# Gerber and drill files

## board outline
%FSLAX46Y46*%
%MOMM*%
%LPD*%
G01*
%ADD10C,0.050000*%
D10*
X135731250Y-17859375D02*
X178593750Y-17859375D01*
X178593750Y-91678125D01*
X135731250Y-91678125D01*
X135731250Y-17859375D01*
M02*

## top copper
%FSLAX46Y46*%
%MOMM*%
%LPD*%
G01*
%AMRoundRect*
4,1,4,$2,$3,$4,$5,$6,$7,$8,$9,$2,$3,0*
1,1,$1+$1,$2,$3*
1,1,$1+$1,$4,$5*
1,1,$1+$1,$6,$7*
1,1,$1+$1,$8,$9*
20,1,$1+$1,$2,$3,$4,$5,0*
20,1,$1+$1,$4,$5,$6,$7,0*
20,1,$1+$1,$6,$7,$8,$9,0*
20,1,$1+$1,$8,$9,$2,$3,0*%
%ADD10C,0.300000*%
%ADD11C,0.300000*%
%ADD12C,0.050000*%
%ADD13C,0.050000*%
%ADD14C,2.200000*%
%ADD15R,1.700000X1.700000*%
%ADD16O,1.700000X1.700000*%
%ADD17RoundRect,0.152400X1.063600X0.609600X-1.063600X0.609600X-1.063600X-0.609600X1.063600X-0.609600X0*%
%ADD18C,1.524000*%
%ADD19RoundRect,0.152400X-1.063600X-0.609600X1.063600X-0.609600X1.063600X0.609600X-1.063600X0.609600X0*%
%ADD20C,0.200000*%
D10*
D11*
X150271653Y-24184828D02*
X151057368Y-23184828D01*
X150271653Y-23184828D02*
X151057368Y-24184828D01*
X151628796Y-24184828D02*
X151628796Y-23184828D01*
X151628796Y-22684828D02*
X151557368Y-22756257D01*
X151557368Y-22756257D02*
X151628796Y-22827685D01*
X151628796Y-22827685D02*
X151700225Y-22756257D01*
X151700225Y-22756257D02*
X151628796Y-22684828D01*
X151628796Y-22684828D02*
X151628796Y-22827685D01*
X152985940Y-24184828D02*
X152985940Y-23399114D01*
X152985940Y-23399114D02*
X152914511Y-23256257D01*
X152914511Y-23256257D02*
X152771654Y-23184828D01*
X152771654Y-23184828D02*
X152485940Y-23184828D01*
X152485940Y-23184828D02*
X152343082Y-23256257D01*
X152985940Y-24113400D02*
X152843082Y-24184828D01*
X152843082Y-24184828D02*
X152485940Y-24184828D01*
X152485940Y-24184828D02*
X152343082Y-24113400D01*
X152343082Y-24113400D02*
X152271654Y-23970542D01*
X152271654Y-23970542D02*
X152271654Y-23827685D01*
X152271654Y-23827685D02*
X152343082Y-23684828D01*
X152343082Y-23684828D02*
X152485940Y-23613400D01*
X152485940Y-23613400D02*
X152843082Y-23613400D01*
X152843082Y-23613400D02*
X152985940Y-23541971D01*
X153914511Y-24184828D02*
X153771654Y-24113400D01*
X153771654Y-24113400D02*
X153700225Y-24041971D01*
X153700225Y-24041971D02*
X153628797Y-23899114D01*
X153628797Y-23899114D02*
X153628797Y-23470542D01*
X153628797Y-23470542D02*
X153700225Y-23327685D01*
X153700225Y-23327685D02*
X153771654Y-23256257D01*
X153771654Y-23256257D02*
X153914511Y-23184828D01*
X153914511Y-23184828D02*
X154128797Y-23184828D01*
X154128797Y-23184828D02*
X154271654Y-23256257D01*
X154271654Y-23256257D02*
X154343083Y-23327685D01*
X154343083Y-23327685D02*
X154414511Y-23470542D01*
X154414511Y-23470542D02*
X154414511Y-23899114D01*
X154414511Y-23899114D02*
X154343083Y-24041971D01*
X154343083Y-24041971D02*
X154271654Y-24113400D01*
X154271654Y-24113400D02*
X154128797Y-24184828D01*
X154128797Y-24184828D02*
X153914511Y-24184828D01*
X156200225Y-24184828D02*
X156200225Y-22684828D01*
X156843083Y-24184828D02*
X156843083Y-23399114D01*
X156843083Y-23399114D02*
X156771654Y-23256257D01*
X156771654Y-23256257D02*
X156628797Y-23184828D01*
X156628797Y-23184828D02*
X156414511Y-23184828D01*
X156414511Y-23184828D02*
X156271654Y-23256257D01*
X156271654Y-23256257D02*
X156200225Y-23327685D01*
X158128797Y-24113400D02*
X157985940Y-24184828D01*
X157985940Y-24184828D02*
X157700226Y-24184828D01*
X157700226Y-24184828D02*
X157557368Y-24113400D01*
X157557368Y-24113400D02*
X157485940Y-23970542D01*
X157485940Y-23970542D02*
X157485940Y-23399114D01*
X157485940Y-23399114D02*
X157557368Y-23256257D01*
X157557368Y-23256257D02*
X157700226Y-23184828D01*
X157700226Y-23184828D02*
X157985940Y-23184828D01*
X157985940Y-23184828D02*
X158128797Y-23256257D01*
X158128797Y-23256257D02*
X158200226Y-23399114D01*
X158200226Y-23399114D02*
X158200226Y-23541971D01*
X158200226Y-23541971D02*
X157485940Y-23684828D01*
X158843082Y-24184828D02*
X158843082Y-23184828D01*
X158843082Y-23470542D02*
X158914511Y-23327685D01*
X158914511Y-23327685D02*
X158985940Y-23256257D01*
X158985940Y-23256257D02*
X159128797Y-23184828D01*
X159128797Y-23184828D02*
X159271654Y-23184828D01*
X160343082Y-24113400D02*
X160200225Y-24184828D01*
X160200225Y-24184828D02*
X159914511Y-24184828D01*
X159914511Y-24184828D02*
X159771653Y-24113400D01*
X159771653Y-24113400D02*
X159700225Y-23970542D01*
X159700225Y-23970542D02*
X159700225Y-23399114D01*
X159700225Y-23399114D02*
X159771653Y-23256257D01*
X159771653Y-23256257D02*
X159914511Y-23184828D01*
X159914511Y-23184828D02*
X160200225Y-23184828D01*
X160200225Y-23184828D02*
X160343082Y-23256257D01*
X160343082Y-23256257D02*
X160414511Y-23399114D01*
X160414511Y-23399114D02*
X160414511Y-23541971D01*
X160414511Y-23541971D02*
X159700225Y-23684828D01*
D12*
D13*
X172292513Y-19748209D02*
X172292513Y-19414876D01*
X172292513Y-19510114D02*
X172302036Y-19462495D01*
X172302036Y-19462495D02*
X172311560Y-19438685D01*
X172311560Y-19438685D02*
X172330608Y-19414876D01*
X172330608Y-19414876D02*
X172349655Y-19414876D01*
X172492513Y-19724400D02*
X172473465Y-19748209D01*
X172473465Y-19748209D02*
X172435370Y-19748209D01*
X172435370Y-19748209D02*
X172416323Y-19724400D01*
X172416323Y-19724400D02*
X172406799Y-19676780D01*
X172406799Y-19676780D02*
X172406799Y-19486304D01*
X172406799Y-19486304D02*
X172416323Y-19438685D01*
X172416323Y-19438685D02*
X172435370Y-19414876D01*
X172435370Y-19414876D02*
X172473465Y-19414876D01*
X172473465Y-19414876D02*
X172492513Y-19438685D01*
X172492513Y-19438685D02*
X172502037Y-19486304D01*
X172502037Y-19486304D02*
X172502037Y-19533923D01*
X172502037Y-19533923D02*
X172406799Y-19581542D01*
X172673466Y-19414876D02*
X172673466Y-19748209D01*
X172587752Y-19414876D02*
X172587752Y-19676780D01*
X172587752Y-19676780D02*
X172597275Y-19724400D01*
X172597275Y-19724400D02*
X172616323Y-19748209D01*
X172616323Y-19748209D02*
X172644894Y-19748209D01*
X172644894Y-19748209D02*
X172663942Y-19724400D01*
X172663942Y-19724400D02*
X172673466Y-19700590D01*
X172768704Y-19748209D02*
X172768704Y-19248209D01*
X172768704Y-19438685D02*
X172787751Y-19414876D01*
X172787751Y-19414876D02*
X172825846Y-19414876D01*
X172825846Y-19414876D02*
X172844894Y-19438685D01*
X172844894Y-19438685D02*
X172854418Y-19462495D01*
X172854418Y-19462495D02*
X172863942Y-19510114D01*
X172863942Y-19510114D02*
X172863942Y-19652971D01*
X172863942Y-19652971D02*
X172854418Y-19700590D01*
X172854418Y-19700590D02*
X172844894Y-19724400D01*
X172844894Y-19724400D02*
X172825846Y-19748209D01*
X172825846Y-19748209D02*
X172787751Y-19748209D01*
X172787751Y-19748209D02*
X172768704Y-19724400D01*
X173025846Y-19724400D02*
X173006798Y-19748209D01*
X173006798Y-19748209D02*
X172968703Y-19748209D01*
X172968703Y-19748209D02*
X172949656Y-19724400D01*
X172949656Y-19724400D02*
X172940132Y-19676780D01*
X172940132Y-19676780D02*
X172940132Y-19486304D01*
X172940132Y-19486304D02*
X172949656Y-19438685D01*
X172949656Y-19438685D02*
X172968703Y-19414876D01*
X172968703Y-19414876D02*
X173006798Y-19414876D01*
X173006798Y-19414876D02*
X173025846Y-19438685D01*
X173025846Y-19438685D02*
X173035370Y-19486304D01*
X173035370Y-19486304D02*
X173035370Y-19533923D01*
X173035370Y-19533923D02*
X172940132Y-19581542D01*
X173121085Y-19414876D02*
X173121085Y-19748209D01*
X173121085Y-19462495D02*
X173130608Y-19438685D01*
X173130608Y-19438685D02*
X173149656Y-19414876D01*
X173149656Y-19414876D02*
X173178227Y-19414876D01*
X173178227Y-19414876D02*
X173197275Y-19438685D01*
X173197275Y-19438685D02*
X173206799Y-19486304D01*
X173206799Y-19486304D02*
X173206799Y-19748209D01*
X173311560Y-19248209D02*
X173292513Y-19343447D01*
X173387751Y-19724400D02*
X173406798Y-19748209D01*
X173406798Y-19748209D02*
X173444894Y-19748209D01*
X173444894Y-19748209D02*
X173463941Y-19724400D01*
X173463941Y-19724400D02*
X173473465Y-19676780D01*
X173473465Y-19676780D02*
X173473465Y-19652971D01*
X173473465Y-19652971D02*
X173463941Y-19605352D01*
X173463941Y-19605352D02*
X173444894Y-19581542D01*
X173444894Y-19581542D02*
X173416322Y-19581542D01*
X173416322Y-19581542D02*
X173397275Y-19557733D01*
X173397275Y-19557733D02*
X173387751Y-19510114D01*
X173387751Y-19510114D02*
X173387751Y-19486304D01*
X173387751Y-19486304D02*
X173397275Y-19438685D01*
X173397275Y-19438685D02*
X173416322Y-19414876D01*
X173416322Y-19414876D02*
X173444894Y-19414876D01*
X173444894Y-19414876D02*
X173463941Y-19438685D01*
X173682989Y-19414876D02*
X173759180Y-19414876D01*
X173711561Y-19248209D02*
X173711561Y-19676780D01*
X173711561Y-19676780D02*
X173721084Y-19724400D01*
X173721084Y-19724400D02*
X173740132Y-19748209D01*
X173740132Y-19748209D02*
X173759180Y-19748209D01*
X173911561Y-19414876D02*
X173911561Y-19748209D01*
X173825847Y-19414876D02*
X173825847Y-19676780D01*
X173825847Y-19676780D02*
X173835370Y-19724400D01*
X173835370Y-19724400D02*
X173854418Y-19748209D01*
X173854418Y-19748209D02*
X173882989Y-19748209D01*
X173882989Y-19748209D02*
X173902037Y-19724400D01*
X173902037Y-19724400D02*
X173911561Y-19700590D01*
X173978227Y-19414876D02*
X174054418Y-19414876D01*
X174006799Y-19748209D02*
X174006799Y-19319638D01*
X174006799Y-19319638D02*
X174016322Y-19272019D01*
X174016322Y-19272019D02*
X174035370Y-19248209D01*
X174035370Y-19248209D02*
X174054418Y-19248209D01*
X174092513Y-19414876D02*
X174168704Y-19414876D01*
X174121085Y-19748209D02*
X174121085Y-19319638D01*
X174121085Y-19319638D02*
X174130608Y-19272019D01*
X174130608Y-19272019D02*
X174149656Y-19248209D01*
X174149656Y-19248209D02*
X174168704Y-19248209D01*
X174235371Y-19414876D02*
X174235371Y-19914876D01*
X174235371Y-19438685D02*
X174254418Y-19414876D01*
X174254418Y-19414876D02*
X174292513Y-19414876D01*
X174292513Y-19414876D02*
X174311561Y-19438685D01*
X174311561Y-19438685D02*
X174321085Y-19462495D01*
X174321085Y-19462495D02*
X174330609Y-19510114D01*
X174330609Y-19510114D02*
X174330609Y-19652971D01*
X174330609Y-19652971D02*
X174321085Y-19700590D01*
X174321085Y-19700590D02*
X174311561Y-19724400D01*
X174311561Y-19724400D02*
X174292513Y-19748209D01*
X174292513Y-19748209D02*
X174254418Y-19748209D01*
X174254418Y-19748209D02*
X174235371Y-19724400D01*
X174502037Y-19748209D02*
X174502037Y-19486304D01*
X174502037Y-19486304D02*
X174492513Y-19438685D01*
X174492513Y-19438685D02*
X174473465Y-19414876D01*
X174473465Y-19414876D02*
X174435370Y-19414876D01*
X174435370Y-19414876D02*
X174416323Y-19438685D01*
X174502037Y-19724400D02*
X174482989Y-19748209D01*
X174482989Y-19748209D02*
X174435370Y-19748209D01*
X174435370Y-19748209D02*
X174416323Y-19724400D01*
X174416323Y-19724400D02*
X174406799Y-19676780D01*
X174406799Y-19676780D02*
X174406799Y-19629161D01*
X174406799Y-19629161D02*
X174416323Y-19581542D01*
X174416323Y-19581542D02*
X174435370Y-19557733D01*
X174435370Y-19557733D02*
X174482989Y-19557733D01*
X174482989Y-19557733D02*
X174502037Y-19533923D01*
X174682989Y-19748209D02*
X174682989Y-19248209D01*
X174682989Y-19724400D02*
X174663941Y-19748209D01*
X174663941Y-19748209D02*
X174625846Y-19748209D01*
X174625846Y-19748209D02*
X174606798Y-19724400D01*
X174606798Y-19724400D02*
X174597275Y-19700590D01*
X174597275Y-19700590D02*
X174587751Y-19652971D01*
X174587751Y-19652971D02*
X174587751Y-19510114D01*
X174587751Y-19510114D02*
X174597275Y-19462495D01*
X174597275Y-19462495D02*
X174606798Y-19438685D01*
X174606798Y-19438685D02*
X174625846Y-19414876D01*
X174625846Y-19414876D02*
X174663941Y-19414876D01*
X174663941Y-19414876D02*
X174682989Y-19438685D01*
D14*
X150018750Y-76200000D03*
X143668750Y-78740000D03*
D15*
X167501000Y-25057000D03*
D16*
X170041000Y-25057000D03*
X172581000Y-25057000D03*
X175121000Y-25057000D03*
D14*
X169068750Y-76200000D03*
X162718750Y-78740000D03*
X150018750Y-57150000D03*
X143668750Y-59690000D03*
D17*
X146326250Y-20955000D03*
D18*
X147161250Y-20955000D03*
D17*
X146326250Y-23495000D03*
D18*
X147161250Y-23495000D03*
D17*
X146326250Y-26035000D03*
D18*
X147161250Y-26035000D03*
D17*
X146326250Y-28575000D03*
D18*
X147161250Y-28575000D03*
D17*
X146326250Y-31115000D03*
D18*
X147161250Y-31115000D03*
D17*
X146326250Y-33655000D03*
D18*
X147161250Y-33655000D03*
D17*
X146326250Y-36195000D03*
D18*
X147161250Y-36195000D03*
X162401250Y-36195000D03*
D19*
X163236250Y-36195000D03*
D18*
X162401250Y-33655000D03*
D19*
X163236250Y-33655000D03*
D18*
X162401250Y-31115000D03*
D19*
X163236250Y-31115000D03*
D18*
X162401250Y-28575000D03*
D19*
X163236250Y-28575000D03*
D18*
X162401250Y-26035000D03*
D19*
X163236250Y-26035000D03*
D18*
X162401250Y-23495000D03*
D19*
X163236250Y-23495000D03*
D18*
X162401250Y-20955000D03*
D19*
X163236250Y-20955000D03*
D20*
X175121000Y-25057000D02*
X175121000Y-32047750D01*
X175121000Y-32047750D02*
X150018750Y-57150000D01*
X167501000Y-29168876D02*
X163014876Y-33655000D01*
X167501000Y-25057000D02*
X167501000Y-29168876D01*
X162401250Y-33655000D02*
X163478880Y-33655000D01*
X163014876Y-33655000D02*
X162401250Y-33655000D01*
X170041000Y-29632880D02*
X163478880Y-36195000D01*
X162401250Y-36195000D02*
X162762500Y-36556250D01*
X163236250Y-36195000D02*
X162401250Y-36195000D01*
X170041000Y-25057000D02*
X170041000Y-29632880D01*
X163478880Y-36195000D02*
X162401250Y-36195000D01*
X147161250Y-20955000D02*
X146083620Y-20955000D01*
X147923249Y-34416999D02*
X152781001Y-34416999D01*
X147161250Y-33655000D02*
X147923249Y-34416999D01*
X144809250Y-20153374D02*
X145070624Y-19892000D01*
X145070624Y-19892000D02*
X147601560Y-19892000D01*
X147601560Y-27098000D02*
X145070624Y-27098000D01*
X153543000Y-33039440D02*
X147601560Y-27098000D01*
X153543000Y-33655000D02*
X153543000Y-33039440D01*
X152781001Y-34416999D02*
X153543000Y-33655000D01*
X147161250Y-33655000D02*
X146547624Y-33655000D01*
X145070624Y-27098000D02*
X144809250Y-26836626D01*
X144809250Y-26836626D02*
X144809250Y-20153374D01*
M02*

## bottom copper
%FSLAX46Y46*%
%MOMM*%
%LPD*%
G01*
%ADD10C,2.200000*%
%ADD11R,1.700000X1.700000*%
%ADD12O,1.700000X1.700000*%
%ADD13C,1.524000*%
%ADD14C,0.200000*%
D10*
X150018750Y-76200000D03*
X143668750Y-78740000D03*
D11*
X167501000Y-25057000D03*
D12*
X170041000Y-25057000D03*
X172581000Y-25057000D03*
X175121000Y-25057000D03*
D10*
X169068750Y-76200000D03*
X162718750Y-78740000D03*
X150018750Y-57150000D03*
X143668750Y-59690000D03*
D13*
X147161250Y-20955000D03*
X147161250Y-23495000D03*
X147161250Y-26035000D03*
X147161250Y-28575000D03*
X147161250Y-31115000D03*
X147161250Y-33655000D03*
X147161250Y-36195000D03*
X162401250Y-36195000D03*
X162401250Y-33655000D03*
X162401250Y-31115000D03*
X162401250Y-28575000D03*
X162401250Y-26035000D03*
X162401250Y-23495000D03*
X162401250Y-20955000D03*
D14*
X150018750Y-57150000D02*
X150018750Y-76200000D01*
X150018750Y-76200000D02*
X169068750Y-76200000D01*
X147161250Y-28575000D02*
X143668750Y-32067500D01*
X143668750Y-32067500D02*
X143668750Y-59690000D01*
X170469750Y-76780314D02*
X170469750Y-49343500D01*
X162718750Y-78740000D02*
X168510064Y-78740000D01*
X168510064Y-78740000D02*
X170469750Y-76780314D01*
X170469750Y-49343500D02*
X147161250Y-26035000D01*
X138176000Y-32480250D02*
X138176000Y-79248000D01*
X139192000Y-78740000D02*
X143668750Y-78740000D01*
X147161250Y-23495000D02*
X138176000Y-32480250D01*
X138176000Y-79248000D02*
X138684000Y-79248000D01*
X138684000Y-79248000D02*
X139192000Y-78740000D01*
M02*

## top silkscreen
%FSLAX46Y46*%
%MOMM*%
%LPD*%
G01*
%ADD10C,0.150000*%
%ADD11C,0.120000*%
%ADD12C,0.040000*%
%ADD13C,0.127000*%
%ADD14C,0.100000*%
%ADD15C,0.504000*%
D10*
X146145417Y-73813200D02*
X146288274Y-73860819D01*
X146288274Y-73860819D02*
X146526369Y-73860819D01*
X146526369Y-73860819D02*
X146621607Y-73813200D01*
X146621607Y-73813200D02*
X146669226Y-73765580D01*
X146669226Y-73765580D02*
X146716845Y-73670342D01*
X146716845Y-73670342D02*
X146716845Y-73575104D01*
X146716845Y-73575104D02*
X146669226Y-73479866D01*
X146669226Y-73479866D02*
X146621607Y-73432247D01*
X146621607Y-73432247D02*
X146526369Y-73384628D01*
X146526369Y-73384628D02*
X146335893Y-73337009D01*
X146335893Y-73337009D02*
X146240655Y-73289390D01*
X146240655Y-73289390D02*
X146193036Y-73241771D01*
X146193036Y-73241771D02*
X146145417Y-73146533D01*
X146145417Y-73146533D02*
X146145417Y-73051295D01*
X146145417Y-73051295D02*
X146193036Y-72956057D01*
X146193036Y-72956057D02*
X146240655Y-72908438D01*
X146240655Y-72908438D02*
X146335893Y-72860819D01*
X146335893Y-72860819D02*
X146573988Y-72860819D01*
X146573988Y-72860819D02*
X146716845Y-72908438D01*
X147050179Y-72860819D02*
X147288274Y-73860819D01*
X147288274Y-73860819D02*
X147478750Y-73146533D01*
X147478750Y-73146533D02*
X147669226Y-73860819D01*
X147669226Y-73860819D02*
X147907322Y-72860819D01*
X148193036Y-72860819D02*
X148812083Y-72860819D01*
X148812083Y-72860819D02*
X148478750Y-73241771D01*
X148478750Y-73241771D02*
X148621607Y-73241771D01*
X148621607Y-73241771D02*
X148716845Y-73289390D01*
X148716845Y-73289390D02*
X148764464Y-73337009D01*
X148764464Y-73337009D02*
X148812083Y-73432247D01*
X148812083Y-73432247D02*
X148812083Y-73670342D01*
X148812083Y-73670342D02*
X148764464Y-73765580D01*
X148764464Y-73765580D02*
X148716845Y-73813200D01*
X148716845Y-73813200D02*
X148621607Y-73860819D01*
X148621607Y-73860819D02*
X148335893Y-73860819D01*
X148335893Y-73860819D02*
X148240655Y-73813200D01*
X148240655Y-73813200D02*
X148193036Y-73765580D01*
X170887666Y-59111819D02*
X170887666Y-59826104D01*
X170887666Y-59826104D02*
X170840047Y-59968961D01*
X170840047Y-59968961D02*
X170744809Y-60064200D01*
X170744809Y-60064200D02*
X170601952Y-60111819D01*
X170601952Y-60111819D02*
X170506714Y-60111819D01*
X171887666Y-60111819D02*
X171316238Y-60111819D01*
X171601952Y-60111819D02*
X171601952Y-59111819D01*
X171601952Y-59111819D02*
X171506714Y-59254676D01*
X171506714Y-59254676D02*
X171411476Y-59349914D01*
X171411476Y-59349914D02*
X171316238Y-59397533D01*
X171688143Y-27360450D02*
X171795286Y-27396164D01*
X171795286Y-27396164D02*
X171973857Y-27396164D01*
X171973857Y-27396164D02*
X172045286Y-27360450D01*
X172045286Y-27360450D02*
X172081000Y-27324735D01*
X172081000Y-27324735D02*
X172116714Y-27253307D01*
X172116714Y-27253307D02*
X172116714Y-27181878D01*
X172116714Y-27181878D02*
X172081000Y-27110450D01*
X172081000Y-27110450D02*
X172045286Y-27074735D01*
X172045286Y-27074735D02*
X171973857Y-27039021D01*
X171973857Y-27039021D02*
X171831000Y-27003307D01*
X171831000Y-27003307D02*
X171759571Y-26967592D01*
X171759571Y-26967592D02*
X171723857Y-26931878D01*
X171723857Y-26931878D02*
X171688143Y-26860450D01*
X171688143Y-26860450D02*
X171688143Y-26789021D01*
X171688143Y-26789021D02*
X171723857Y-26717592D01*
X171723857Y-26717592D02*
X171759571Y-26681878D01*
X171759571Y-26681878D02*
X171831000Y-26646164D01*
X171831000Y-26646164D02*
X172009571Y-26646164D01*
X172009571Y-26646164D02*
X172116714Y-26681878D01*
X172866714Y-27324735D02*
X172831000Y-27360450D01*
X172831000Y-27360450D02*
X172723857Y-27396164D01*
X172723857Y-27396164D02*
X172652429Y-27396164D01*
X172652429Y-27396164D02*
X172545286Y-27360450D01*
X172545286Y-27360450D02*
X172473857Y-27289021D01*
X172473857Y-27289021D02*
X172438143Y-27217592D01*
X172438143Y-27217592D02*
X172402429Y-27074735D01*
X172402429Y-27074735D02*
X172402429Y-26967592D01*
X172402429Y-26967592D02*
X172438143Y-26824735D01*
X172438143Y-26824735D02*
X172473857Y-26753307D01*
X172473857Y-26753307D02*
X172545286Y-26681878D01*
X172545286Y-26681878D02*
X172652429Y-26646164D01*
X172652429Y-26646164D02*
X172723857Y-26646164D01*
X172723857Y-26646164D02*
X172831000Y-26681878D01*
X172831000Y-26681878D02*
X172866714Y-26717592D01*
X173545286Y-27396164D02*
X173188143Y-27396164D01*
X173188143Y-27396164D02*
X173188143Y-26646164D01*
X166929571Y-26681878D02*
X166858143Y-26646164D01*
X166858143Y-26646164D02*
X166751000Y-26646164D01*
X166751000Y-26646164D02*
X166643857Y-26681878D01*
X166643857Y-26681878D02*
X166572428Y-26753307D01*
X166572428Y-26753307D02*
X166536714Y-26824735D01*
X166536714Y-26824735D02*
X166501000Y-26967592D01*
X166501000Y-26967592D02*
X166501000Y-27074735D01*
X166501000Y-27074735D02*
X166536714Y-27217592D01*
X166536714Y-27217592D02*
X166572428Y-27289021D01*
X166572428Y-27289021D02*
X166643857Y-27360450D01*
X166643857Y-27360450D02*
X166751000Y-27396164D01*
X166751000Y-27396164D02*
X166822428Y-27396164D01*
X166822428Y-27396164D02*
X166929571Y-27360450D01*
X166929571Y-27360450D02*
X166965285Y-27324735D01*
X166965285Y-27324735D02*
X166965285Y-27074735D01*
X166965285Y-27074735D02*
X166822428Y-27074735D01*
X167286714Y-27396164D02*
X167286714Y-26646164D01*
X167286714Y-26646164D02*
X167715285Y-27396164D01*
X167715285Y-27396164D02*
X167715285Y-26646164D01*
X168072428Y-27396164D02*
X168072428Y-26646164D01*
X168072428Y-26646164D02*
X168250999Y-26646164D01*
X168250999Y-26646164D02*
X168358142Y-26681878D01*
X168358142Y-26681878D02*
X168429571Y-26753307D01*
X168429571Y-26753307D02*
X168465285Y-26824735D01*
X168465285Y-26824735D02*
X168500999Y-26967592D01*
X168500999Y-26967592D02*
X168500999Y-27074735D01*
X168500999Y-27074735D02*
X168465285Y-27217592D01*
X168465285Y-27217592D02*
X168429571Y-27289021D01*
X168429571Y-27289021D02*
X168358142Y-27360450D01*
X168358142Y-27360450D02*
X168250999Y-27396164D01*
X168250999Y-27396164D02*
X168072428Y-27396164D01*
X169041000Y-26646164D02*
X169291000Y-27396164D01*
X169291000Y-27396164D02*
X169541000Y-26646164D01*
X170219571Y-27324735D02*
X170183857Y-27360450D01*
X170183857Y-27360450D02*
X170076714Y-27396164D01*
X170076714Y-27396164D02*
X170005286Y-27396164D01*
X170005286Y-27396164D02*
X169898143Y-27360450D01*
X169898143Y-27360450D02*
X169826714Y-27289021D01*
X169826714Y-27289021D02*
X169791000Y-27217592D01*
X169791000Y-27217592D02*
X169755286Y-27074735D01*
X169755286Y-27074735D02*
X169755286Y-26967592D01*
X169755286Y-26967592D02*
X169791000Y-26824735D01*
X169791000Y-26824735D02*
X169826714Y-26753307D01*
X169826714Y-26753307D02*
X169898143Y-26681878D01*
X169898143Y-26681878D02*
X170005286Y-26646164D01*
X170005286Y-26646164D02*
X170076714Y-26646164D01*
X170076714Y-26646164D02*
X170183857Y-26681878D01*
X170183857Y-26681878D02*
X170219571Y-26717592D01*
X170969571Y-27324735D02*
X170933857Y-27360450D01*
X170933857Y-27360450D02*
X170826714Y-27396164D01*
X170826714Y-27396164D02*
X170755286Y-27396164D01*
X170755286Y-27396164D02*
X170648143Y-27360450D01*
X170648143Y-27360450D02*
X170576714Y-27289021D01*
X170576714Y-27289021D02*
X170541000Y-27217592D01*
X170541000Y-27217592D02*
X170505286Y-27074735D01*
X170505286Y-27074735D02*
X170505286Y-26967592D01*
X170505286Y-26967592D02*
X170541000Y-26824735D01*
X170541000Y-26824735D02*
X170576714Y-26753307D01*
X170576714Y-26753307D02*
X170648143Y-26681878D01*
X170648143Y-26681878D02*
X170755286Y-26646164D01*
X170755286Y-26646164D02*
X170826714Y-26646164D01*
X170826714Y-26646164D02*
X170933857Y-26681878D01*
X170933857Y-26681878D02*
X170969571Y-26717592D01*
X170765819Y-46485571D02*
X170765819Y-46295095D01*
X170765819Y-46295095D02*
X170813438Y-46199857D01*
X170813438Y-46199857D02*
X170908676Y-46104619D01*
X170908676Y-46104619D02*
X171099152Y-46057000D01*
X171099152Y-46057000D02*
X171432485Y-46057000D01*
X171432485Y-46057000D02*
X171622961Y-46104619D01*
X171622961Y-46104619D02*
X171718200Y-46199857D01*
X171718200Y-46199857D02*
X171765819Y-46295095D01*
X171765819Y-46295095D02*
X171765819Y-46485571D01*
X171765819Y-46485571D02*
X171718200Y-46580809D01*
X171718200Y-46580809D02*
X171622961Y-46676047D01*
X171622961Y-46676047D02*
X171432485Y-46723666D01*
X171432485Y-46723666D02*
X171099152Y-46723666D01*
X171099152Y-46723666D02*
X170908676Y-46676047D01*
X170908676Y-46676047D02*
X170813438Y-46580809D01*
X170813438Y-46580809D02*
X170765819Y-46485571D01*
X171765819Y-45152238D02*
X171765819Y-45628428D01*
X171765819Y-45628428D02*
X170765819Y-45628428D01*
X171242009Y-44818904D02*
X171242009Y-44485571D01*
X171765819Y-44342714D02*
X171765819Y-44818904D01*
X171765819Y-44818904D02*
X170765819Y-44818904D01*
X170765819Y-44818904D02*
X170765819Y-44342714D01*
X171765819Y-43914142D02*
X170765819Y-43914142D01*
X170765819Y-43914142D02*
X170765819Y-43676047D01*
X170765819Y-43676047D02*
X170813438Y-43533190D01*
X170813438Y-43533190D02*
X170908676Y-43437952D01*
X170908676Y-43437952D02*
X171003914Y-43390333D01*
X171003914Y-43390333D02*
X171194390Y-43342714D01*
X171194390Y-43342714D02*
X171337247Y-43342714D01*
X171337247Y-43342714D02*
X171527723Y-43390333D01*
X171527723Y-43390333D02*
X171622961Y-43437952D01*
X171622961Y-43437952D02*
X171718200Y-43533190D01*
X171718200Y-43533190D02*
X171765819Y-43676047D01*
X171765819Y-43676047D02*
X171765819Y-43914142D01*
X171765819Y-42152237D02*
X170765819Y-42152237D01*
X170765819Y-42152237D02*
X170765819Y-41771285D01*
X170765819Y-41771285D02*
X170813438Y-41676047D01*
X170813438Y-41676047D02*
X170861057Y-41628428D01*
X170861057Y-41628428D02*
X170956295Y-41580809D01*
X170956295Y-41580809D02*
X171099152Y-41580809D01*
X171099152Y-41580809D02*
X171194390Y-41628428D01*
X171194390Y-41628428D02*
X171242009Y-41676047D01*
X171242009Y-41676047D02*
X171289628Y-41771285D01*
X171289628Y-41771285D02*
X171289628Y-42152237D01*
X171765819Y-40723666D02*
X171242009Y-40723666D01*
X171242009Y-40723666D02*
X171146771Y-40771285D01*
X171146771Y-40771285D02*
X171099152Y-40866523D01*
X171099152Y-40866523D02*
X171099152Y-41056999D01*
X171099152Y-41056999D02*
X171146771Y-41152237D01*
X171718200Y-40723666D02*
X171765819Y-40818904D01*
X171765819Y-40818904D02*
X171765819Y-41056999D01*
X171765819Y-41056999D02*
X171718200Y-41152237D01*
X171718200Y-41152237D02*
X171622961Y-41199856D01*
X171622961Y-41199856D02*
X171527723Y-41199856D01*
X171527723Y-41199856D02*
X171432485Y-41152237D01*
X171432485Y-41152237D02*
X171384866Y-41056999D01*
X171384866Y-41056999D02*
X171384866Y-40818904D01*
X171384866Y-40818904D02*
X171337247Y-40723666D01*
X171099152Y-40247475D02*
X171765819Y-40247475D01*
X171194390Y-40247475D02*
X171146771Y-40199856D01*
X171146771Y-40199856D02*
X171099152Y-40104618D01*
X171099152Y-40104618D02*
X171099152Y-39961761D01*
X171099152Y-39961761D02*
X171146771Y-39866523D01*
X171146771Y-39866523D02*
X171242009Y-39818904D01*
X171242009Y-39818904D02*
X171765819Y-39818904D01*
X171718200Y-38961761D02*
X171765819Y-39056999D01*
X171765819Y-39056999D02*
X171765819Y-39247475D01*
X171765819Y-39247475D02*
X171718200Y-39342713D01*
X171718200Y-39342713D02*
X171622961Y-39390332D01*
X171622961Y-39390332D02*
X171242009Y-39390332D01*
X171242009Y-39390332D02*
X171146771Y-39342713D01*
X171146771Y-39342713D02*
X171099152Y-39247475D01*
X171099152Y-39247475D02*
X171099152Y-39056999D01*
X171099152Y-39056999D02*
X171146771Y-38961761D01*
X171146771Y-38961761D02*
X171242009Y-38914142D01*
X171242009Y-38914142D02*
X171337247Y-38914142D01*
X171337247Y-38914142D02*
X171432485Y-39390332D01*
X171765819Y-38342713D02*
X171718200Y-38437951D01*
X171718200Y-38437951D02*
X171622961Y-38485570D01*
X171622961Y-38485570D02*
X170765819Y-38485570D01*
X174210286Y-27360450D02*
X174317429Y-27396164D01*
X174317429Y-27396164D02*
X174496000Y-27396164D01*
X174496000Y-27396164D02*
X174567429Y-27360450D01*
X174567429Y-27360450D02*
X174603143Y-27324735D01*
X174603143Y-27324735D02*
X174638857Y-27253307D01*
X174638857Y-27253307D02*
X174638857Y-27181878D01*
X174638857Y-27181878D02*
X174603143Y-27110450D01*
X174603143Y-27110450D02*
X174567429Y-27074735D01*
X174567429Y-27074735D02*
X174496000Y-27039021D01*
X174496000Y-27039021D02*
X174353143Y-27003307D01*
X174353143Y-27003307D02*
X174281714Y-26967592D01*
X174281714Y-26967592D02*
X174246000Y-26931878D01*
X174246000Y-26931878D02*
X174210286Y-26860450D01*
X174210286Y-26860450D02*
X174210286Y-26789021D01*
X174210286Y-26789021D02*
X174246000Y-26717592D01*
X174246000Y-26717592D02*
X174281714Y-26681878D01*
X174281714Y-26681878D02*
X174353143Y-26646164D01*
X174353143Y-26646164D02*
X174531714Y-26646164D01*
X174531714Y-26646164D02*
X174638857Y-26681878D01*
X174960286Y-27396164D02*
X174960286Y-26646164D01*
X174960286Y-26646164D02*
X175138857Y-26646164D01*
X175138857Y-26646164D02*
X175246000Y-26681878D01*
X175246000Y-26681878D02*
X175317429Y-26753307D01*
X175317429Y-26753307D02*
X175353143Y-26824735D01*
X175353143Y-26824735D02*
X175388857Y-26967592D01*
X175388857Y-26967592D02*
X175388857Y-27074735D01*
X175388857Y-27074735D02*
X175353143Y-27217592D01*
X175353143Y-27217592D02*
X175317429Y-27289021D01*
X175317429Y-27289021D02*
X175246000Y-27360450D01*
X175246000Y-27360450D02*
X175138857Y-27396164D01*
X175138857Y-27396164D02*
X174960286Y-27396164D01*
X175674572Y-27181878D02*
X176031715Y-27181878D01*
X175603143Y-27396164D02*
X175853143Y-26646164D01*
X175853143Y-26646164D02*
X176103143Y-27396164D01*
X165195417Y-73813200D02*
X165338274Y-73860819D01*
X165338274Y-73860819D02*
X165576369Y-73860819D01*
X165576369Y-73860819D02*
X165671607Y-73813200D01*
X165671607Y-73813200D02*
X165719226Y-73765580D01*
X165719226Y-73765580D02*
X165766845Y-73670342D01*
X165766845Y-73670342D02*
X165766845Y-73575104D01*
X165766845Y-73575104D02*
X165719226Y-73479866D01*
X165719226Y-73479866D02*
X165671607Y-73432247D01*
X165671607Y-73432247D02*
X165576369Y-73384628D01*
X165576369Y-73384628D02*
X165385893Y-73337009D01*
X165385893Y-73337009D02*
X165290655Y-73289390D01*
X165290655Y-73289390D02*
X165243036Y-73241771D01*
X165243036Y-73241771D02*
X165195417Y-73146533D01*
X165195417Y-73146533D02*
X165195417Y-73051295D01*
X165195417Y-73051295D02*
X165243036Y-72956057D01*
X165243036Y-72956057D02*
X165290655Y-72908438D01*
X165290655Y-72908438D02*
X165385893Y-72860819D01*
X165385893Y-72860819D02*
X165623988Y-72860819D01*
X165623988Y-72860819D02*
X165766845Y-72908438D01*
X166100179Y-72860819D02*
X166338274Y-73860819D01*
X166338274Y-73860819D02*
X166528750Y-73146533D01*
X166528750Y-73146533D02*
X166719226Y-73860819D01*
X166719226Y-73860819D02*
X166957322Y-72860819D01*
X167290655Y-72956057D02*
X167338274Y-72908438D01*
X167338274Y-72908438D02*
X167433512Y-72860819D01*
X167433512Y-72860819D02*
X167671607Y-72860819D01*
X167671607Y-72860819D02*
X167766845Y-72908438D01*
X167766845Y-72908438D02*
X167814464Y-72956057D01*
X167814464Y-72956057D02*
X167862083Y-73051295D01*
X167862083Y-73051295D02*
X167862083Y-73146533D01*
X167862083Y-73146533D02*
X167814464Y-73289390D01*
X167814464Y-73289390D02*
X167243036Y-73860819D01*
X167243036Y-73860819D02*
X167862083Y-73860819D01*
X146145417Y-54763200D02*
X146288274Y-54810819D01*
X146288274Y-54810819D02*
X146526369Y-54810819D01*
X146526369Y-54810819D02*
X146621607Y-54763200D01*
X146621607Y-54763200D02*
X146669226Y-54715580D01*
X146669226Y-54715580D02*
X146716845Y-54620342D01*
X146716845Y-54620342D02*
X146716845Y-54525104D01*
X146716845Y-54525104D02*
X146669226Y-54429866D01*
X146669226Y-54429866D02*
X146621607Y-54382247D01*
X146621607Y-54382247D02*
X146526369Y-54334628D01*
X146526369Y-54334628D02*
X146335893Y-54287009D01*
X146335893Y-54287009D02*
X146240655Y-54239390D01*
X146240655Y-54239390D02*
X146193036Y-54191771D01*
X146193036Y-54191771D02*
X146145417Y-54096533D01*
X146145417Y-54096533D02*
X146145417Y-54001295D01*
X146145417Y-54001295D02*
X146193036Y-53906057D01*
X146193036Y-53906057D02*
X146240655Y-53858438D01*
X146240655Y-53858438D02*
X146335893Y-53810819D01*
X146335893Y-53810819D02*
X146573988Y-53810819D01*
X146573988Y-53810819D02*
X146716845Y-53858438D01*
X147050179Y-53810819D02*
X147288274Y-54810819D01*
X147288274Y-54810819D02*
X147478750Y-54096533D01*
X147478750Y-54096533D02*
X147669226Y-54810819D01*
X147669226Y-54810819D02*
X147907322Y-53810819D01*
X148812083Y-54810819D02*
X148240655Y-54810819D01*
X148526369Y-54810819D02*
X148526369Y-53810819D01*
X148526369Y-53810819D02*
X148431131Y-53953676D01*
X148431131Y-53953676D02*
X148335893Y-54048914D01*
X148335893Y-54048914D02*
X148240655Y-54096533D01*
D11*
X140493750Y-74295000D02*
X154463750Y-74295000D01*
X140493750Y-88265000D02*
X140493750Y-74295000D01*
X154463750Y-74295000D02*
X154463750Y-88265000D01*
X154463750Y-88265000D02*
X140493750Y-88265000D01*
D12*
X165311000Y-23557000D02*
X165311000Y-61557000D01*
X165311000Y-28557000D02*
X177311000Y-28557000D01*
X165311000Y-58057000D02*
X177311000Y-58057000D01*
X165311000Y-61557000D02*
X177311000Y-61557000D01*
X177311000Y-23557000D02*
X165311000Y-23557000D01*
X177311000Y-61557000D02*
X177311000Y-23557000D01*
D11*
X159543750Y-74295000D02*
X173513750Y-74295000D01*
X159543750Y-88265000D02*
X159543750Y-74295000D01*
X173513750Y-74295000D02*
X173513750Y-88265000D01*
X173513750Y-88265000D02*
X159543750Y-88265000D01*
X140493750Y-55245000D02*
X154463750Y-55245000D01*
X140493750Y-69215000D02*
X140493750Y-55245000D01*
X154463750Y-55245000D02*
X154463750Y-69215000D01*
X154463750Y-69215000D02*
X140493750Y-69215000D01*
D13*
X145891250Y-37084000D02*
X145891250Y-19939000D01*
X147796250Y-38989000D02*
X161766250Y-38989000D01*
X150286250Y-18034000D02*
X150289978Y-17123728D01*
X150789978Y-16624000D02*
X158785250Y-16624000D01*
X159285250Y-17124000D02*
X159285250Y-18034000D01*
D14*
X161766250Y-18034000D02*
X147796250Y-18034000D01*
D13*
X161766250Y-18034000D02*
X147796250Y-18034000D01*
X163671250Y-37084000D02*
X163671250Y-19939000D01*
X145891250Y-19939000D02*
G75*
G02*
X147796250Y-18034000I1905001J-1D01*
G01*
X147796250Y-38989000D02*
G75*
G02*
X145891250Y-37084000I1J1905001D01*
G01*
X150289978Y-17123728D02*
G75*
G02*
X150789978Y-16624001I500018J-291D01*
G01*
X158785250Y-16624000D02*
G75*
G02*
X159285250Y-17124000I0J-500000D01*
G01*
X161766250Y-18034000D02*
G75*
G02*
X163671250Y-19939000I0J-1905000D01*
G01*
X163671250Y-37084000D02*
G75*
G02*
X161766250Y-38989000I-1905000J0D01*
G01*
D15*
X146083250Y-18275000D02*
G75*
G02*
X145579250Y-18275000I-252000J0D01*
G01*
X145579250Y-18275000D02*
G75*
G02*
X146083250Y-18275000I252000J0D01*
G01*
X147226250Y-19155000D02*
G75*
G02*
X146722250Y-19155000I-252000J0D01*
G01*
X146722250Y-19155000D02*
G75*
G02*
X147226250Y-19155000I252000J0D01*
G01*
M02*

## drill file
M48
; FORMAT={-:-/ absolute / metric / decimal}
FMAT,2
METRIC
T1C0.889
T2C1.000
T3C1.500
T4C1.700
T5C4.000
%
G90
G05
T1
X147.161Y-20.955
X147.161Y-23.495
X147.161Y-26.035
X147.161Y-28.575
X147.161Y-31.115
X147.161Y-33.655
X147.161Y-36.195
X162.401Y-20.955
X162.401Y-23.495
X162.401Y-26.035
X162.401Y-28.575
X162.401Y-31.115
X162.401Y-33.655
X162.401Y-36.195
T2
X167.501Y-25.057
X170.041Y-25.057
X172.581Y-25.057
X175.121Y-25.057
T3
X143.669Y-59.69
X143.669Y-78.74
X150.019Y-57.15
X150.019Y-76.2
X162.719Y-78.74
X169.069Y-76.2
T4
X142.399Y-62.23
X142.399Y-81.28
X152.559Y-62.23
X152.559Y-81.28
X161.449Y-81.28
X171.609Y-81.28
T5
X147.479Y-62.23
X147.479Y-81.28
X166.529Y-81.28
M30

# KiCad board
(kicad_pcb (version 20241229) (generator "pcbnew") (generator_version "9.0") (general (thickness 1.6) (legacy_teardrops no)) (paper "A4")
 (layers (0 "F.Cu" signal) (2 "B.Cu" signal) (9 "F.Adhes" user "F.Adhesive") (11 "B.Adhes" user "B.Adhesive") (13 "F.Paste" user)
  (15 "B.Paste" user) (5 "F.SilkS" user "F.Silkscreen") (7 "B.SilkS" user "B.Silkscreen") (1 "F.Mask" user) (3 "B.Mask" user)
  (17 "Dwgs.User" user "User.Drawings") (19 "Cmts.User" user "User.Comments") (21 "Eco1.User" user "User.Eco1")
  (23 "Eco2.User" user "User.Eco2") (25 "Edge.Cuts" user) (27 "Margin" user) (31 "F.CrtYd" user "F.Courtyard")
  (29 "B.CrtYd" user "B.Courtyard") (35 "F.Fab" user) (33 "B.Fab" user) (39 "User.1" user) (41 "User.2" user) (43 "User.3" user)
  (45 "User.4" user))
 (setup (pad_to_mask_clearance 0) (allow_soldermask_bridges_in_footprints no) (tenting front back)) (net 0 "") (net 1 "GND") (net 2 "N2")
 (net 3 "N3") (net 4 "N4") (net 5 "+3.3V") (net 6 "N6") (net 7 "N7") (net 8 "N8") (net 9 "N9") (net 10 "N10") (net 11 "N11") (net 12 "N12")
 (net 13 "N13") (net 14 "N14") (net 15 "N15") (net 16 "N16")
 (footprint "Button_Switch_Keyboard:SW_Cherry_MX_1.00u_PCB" (layer "F.Cu") (at 150.01875 76.2)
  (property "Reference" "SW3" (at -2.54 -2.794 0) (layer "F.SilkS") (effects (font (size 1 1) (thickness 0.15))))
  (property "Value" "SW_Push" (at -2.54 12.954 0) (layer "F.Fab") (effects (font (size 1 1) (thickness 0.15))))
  (fp_line (start -9.525 -1.905) (end 4.445 -1.905) (stroke (width 0.12) (type solid)) (layer "F.SilkS"))
  (fp_line (start -9.525 12.065) (end -9.525 -1.905) (stroke (width 0.12) (type solid)) (layer "F.SilkS"))
  (fp_line (start 4.445 -1.905) (end 4.445 12.065) (stroke (width 0.12) (type solid)) (layer "F.SilkS"))
  (fp_line (start 4.445 12.065) (end -9.525 12.065) (stroke (width 0.12) (type solid)) (layer "F.SilkS"))
  (pad "" np_thru_hole circle (at -7.62 5.08) (size 1.7 1.7) (drill 1.7) (layers "*.Cu" "*.Mask"))
  (pad "" np_thru_hole circle (at -2.54 5.08) (size 4 4) (drill 4) (layers "*.Cu" "*.Mask"))
  (pad "" np_thru_hole circle (at 2.54 5.08) (size 1.7 1.7) (drill 1.7) (layers "*.Cu" "*.Mask"))
  (pad "1" thru_hole circle (at 0 0) (size 2.2 2.2) (drill 1.5) (layers "*.Cu" "*.Mask") (remove_unused_layers no) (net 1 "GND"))
  (pad "2" thru_hole circle (at -6.35 2.54) (size 2.2 2.2) (drill 1.5) (layers "*.Cu" "*.Mask") (remove_unused_layers no) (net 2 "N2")))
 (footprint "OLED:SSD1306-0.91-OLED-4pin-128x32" (layer "F.Cu") (at 165.311 61.557 90)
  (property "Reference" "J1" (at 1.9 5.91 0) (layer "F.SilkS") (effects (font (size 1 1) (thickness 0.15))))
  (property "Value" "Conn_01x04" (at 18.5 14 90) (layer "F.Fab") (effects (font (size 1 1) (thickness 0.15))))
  (fp_line (start 38 0) (end 0 0) (stroke (width 0.04) (type solid)) (layer "F.SilkS"))
  (fp_line (start 33 0) (end 33 12) (stroke (width 0.04) (type solid)) (layer "F.SilkS"))
  (fp_line (start 3.5 0) (end 3.5 12) (stroke (width 0.04) (type solid)) (layer "F.SilkS"))
  (fp_line (start 0 0) (end 0 12) (stroke (width 0.04) (type solid)) (layer "F.SilkS"))
  (fp_line (start 38 12) (end 38 0) (stroke (width 0.04) (type solid)) (layer "F.SilkS"))
  (fp_line (start 0 12) (end 38 12) (stroke (width 0.04) (type solid)) (layer "F.SilkS"))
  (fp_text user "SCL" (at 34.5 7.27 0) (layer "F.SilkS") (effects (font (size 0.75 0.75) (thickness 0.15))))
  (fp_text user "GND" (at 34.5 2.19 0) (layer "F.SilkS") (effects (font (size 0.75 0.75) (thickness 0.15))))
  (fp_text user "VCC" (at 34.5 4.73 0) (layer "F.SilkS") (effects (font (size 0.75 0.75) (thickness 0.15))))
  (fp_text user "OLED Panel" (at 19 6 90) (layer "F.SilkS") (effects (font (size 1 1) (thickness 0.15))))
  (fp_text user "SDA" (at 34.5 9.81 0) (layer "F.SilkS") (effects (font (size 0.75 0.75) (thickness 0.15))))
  (pad "1" thru_hole rect (at 36.5 2.19 90) (size 1.7 1.7) (drill 1) (layers "*.Cu" "*.Mask") (remove_unused_layers no) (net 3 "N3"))
  (pad "2" thru_hole oval (at 36.5 4.73 90) (size 1.7 1.7) (drill 1) (layers "*.Cu" "*.Mask") (remove_unused_layers no) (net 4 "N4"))
  (pad "3" thru_hole oval (at 36.5 7.27 90) (size 1.7 1.7) (drill 1) (layers "*.Cu" "*.Mask") (remove_unused_layers no) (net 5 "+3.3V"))
  (pad "4" thru_hole oval (at 36.5 9.81 90) (size 1.7 1.7) (drill 1) (layers "*.Cu" "*.Mask") (remove_unused_layers no) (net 1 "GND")))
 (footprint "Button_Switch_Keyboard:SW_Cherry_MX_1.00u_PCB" (layer "F.Cu") (at 169.06875 76.2)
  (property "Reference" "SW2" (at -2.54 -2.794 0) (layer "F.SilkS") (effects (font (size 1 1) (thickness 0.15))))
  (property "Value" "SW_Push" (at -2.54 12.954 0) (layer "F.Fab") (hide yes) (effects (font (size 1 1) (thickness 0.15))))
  (fp_line (start -9.525 -1.905) (end 4.445 -1.905) (stroke (width 0.12) (type solid)) (layer "F.SilkS"))
  (fp_line (start -9.525 12.065) (end -9.525 -1.905) (stroke (width 0.12) (type solid)) (layer "F.SilkS"))
  (fp_line (start 4.445 -1.905) (end 4.445 12.065) (stroke (width 0.12) (type solid)) (layer "F.SilkS"))
  (fp_line (start 4.445 12.065) (end -9.525 12.065) (stroke (width 0.12) (type solid)) (layer "F.SilkS"))
  (pad "" np_thru_hole circle (at -7.62 5.08) (size 1.7 1.7) (drill 1.7) (layers "*.Cu" "*.Mask"))
  (pad "" np_thru_hole circle (at -2.54 5.08) (size 4 4) (drill 4) (layers "*.Cu" "*.Mask"))
  (pad "" np_thru_hole circle (at 2.54 5.08) (size 1.7 1.7) (drill 1.7) (layers "*.Cu" "*.Mask"))
  (pad "1" thru_hole circle (at 0 0) (size 2.2 2.2) (drill 1.5) (layers "*.Cu" "*.Mask") (remove_unused_layers no) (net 1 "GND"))
  (pad "2" thru_hole circle (at -6.35 2.54) (size 2.2 2.2) (drill 1.5) (layers "*.Cu" "*.Mask") (remove_unused_layers no) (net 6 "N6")))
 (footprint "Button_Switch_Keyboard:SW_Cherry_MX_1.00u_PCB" (layer "F.Cu") (at 150.01875 57.15)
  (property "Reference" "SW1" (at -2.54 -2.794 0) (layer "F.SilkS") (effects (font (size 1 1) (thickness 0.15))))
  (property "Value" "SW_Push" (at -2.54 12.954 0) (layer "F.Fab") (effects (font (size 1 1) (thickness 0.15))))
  (fp_line (start -9.525 -1.905) (end 4.445 -1.905) (stroke (width 0.12) (type solid)) (layer "F.SilkS"))
  (fp_line (start -9.525 12.065) (end -9.525 -1.905) (stroke (width 0.12) (type solid)) (layer "F.SilkS"))
  (fp_line (start 4.445 -1.905) (end 4.445 12.065) (stroke (width 0.12) (type solid)) (layer "F.SilkS"))
  (fp_line (start 4.445 12.065) (end -9.525 12.065) (stroke (width 0.12) (type solid)) (layer "F.SilkS"))
  (pad "" np_thru_hole circle (at -7.62 5.08) (size 1.7 1.7) (drill 1.7) (layers "*.Cu" "*.Mask"))
  (pad "" np_thru_hole circle (at -2.54 5.08) (size 4 4) (drill 4) (layers "*.Cu" "*.Mask"))
  (pad "" np_thru_hole circle (at 2.54 5.08) (size 1.7 1.7) (drill 1.7) (layers "*.Cu" "*.Mask"))
  (pad "1" thru_hole circle (at 0 0) (size 2.2 2.2) (drill 1.5) (layers "*.Cu" "*.Mask") (remove_unused_layers no) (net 1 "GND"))
  (pad "2" thru_hole circle (at -6.35 2.54) (size 2.2 2.2) (drill 1.5) (layers "*.Cu" "*.Mask") (remove_unused_layers no) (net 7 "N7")))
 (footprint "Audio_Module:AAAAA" (layer "F.Cu") (at 154.78125 28.575)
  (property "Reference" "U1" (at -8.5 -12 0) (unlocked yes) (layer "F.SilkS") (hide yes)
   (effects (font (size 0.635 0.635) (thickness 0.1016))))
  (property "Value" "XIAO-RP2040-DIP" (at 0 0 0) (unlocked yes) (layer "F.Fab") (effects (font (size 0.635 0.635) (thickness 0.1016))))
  (fp_line (start -8.89 8.509) (end -8.89 -8.636) (stroke (width 0.127) (type solid)) (layer "F.SilkS"))
  (fp_line (start -6.985 10.414) (end 6.985 10.414) (stroke (width 0.127) (type solid)) (layer "F.SilkS"))
  (fp_line (start -4.495 -10.541) (end -4.491272 -11.451272) (stroke (width 0.127) (type solid)) (layer "F.SilkS"))
  (fp_line (start -3.991272 -11.951) (end 4.004 -11.951) (stroke (width 0.127) (type solid)) (layer "F.SilkS"))
  (fp_line (start 4.504 -11.451) (end 4.504 -10.541) (stroke (width 0.127) (type solid)) (layer "F.SilkS"))
  (fp_line (start 6.985 -10.541) (end -6.985 -10.541) (stroke (width 0.1) (type solid)) (layer "F.SilkS"))
  (fp_line (start 6.985 -10.541) (end -6.985 -10.541) (stroke (width 0.127) (type solid)) (layer "F.SilkS"))
  (fp_line (start 8.89 8.509) (end 8.89 -8.636) (stroke (width 0.127) (type solid)) (layer "F.SilkS"))
  (fp_arc (start -8.89 -8.636) (mid -8.332038 -9.983038) (end -6.985 -10.541) (stroke (width 0.127) (type solid)) (layer "F.SilkS"))
  (fp_arc (start -6.985 10.414) (mid -8.332038 9.856038) (end -8.89 8.509) (stroke (width 0.127) (type solid)) (layer "F.SilkS"))
  (fp_arc (start -4.491272 -11.451272) (mid -4.344728 -11.80464) (end -3.991272 -11.951) (stroke (width 0.127) (type default))
   (layer "F.SilkS"))
  (fp_arc (start 4.004 -11.951) (mid 4.357553 -11.804553) (end 4.504 -11.451) (stroke (width 0.127) (type default)) (layer "F.SilkS"))
  (fp_arc (start 6.985 -10.541) (mid 8.332038 -9.983038) (end 8.89 -8.636) (stroke (width 0.127) (type solid)) (layer "F.SilkS"))
  (fp_arc (start 8.89 8.509) (mid 8.332038 9.856038) (end 6.985 10.414) (stroke (width 0.127) (type solid)) (layer "F.SilkS"))
  (fp_circle (center -8.95 -10.3) (end -8.95 -10.554) (stroke (width 0.5) (type solid)) (fill yes) (layer "F.SilkS"))
  (fp_circle (center -7.807 -9.42) (end -7.807 -9.674) (stroke (width 0.5) (type solid)) (fill yes) (layer "F.SilkS"))
  (pad "1" smd roundrect (at -8.455 -7.62 180) (size 2.432 1.524) (layers "F.Cu" "F.Mask") (roundrect_rratio 0.1) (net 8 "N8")
   (thermal_bridge_angle 45))
  (pad "1" thru_hole circle (at -7.62 -7.62 180) (size 1.524 1.524) (drill 0.889) (layers "*.Cu" "*.Mask") (remove_unused_layers no)
   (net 8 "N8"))
  (pad "2" smd roundrect (at -8.455 -5.08 180) (size 2.432 1.524) (layers "F.Cu" "F.Mask") (roundrect_rratio 0.1) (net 2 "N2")
   (thermal_bridge_angle 45))
  (pad "2" thru_hole circle (at -7.62 -5.08 180) (size 1.524 1.524) (drill 0.889) (layers "*.Cu" "*.Mask") (remove_unused_layers no)
   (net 2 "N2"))
  (pad "3" smd roundrect (at -8.455 -2.54 180) (size 2.432 1.524) (layers "F.Cu" "F.Mask") (roundrect_rratio 0.1) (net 6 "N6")
   (thermal_bridge_angle 45))
  (pad "3" thru_hole circle (at -7.62 -2.54 180) (size 1.524 1.524) (drill 0.889) (layers "*.Cu" "*.Mask") (remove_unused_layers no)
   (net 6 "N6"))
  (pad "4" smd roundrect (at -8.455 0 180) (size 2.432 1.524) (layers "F.Cu" "F.Mask") (roundrect_rratio 0.1) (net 7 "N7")
   (thermal_bridge_angle 45))
  (pad "4" thru_hole circle (at -7.62 0 180) (size 1.524 1.524) (drill 0.889) (layers "*.Cu" "*.Mask") (remove_unused_layers no)
   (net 7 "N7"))
  (pad "5" smd roundrect (at -8.455 2.54 180) (size 2.432 1.524) (layers "F.Cu" "F.Mask") (roundrect_rratio 0.1) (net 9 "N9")
   (thermal_bridge_angle 45))
  (pad "5" thru_hole circle (at -7.62 2.54 180) (size 1.524 1.524) (drill 0.889) (layers "*.Cu" "*.Mask") (remove_unused_layers no)
   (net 9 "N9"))
  (pad "6" smd roundrect (at -8.455 5.08 180) (size 2.432 1.524) (layers "F.Cu" "F.Mask") (roundrect_rratio 0.1) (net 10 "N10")
   (thermal_bridge_angle 45))
  (pad "6" thru_hole circle (at -7.62 5.08 180) (size 1.524 1.524) (drill 0.889) (layers "*.Cu" "*.Mask") (remove_unused_layers no)
   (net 10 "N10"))
  (pad "7" smd roundrect (at -8.455 7.62 180) (size 2.432 1.524) (layers "F.Cu" "F.Mask") (roundrect_rratio 0.1) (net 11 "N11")
   (thermal_bridge_angle 45))
  (pad "7" thru_hole circle (at -7.62 7.62 180) (size 1.524 1.524) (drill 0.889) (layers "*.Cu" "*.Mask") (remove_unused_layers no)
   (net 11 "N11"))
  (pad "8" thru_hole circle (at 7.62 7.62) (size 1.524 1.524) (drill 0.889) (layers "*.Cu" "*.Mask") (remove_unused_layers no) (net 4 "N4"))
  (pad "8" smd roundrect (at 8.455 7.62) (size 2.432 1.524) (layers "F.Cu" "F.Mask") (roundrect_rratio 0.1) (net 4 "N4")
   (thermal_bridge_angle 45))
  (pad "9" thru_hole circle (at 7.62 5.08) (size 1.524 1.524) (drill 0.889) (layers "*.Cu" "*.Mask") (remove_unused_layers no) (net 3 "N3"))
  (pad "9" smd roundrect (at 8.455 5.08) (size 2.432 1.524) (layers "F.Cu" "F.Mask") (roundrect_rratio 0.1) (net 3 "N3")
   (thermal_bridge_angle 45))
  (pad "10" thru_hole circle (at 7.62 2.54) (size 1.524 1.524) (drill 0.889) (layers "*.Cu" "*.Mask") (remove_unused_layers no)
   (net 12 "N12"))
  (pad "10" smd roundrect (at 8.455 2.54) (size 2.432 1.524) (layers "F.Cu" "F.Mask") (roundrect_rratio 0.1) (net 12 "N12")
   (thermal_bridge_angle 45))
  (pad "11" thru_hole circle (at 7.62 0) (size 1.524 1.524) (drill 0.889) (layers "*.Cu" "*.Mask") (remove_unused_layers no) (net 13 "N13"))
  (pad "11" smd roundrect (at 8.455 0) (size 2.432 1.524) (layers "F.Cu" "F.Mask") (roundrect_rratio 0.1) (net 13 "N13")
   (thermal_bridge_angle 45))
  (pad "12" thru_hole circle (at 7.62 -2.54) (size 1.524 1.524) (drill 0.889) (layers "*.Cu" "*.Mask") (remove_unused_layers no)
   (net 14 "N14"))
  (pad "12" smd roundrect (at 8.455 -2.54) (size 2.432 1.524) (layers "F.Cu" "F.Mask") (roundrect_rratio 0.1) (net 14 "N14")
   (thermal_bridge_angle 45))
  (pad "13" thru_hole circle (at 7.62 -5.08) (size 1.524 1.524) (drill 0.889) (layers "*.Cu" "*.Mask") (remove_unused_layers no)
   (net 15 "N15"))
  (pad "13" smd roundrect (at 8.455 -5.08) (size 2.432 1.524) (layers "F.Cu" "F.Mask") (roundrect_rratio 0.1) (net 15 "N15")
   (thermal_bridge_angle 45))
  (pad "14" thru_hole circle (at 7.62 -7.62) (size 1.524 1.524) (drill 0.889) (layers "*.Cu" "*.Mask") (remove_unused_layers no)
   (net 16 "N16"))
  (pad "14" smd roundrect (at 8.455 -7.62) (size 2.432 1.524) (layers "F.Cu" "F.Mask") (roundrect_rratio 0.1) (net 16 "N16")
   (thermal_bridge_angle 45)))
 (gr_rect (start 135.73125 17.859375) (end 178.59375 91.678125) (stroke (width 0.05) (type default)) (fill no) (layer "Edge.Cuts"))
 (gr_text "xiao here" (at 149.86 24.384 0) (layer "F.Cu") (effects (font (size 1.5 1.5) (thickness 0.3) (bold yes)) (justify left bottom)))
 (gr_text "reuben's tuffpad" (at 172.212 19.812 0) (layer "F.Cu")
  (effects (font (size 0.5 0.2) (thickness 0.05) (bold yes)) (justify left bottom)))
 (segment (start 175.121 25.057) (end 175.121 32.04775) (width 0.2) (layer "F.Cu") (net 1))
 (segment (start 175.121 32.04775) (end 150.01875 57.15) (width 0.2) (layer "F.Cu") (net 1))
 (segment (start 150.01875 57.15) (end 150.01875 76.2) (width 0.2) (layer "B.Cu") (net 1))
 (segment (start 150.01875 76.2) (end 169.06875 76.2) (width 0.2) (layer "B.Cu") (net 1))
 (segment (start 147.16125 28.575) (end 143.66875 32.0675) (width 0.2) (layer "B.Cu") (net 7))
 (segment (start 143.66875 32.0675) (end 143.66875 59.69) (width 0.2) (layer "B.Cu") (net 7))
 (segment (start 170.46975 76.780314) (end 170.46975 49.3435) (width 0.2) (layer "B.Cu") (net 6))
 (segment (start 162.71875 78.74) (end 168.510064 78.74) (width 0.2) (layer "B.Cu") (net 6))
 (segment (start 168.510064 78.74) (end 170.46975 76.780314) (width 0.2) (layer "B.Cu") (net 6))
 (segment (start 170.46975 49.3435) (end 147.16125 26.035) (width 0.2) (layer "B.Cu") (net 6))
 (segment (start 138.176 32.48025) (end 138.176 79.248) (width 0.2) (layer "B.Cu") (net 2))
 (segment (start 139.192 78.74) (end 143.66875 78.74) (width 0.2) (layer "B.Cu") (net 2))
 (segment (start 147.16125 23.495) (end 138.176 32.48025) (width 0.2) (layer "B.Cu") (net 2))
 (segment (start 138.176 79.248) (end 138.684 79.248) (width 0.2) (layer "B.Cu") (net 2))
 (segment (start 138.684 79.248) (end 139.192 78.74) (width 0.2) (layer "B.Cu") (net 2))
 (segment (start 167.501 29.168876) (end 163.014876 33.655) (width 0.2) (layer "F.Cu") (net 3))
 (segment (start 167.501 25.057) (end 167.501 29.168876) (width 0.2) (layer "F.Cu") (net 3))
 (segment (start 162.40125 33.655) (end 163.47888 33.655) (width 0.2) (layer "F.Cu") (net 3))
 (segment (start 163.014876 33.655) (end 162.40125 33.655) (width 0.2) (layer "F.Cu") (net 3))
 (segment (start 170.041 29.63288) (end 163.47888 36.195) (width 0.2) (layer "F.Cu") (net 4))
 (segment (start 162.40125 36.195) (end 162.7625 36.55625) (width 0.2) (layer "F.Cu") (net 4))
 (segment (start 163.23625 36.195) (end 162.40125 36.195) (width 0.2) (layer "F.Cu") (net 4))
 (segment (start 170.041 25.057) (end 170.041 29.63288) (width 0.2) (layer "F.Cu") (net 4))
 (segment (start 163.47888 36.195) (end 162.40125 36.195) (width 0.2) (layer "F.Cu") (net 4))
 (segment (start 147.16125 20.955) (end 146.08362 20.955) (width 0.2) (layer "F.Cu") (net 8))
 (segment (start 147.923249 34.416999) (end 152.781001 34.416999) (width 0.2) (layer "F.Cu") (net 10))
 (segment (start 147.16125 33.655) (end 147.923249 34.416999) (width 0.2) (layer "F.Cu") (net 10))
 (segment (start 144.80925 20.153374) (end 145.070624 19.892) (width 0.2) (layer "F.Cu") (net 10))
 (segment (start 145.070624 19.892) (end 147.60156 19.892) (width 0.2) (layer "F.Cu") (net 10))
 (segment (start 147.60156 27.098) (end 145.070624 27.098) (width 0.2) (layer "F.Cu") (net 10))
 (segment (start 153.543 33.03944) (end 147.60156 27.098) (width 0.2) (layer "F.Cu") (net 10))
 (segment (start 153.543 33.655) (end 153.543 33.03944) (width 0.2) (layer "F.Cu") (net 10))
 (segment (start 152.781001 34.416999) (end 153.543 33.655) (width 0.2) (layer "F.Cu") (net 10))
 (segment (start 147.16125 33.655) (end 146.547624 33.655) (width 0.2) (layer "F.Cu") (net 10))
 (segment (start 145.070624 27.098) (end 144.80925 26.836626) (width 0.2) (layer "F.Cu") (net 10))
 (segment (start 144.80925 26.836626) (end 144.80925 20.153374) (width 0.2) (layer "F.Cu") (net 10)))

